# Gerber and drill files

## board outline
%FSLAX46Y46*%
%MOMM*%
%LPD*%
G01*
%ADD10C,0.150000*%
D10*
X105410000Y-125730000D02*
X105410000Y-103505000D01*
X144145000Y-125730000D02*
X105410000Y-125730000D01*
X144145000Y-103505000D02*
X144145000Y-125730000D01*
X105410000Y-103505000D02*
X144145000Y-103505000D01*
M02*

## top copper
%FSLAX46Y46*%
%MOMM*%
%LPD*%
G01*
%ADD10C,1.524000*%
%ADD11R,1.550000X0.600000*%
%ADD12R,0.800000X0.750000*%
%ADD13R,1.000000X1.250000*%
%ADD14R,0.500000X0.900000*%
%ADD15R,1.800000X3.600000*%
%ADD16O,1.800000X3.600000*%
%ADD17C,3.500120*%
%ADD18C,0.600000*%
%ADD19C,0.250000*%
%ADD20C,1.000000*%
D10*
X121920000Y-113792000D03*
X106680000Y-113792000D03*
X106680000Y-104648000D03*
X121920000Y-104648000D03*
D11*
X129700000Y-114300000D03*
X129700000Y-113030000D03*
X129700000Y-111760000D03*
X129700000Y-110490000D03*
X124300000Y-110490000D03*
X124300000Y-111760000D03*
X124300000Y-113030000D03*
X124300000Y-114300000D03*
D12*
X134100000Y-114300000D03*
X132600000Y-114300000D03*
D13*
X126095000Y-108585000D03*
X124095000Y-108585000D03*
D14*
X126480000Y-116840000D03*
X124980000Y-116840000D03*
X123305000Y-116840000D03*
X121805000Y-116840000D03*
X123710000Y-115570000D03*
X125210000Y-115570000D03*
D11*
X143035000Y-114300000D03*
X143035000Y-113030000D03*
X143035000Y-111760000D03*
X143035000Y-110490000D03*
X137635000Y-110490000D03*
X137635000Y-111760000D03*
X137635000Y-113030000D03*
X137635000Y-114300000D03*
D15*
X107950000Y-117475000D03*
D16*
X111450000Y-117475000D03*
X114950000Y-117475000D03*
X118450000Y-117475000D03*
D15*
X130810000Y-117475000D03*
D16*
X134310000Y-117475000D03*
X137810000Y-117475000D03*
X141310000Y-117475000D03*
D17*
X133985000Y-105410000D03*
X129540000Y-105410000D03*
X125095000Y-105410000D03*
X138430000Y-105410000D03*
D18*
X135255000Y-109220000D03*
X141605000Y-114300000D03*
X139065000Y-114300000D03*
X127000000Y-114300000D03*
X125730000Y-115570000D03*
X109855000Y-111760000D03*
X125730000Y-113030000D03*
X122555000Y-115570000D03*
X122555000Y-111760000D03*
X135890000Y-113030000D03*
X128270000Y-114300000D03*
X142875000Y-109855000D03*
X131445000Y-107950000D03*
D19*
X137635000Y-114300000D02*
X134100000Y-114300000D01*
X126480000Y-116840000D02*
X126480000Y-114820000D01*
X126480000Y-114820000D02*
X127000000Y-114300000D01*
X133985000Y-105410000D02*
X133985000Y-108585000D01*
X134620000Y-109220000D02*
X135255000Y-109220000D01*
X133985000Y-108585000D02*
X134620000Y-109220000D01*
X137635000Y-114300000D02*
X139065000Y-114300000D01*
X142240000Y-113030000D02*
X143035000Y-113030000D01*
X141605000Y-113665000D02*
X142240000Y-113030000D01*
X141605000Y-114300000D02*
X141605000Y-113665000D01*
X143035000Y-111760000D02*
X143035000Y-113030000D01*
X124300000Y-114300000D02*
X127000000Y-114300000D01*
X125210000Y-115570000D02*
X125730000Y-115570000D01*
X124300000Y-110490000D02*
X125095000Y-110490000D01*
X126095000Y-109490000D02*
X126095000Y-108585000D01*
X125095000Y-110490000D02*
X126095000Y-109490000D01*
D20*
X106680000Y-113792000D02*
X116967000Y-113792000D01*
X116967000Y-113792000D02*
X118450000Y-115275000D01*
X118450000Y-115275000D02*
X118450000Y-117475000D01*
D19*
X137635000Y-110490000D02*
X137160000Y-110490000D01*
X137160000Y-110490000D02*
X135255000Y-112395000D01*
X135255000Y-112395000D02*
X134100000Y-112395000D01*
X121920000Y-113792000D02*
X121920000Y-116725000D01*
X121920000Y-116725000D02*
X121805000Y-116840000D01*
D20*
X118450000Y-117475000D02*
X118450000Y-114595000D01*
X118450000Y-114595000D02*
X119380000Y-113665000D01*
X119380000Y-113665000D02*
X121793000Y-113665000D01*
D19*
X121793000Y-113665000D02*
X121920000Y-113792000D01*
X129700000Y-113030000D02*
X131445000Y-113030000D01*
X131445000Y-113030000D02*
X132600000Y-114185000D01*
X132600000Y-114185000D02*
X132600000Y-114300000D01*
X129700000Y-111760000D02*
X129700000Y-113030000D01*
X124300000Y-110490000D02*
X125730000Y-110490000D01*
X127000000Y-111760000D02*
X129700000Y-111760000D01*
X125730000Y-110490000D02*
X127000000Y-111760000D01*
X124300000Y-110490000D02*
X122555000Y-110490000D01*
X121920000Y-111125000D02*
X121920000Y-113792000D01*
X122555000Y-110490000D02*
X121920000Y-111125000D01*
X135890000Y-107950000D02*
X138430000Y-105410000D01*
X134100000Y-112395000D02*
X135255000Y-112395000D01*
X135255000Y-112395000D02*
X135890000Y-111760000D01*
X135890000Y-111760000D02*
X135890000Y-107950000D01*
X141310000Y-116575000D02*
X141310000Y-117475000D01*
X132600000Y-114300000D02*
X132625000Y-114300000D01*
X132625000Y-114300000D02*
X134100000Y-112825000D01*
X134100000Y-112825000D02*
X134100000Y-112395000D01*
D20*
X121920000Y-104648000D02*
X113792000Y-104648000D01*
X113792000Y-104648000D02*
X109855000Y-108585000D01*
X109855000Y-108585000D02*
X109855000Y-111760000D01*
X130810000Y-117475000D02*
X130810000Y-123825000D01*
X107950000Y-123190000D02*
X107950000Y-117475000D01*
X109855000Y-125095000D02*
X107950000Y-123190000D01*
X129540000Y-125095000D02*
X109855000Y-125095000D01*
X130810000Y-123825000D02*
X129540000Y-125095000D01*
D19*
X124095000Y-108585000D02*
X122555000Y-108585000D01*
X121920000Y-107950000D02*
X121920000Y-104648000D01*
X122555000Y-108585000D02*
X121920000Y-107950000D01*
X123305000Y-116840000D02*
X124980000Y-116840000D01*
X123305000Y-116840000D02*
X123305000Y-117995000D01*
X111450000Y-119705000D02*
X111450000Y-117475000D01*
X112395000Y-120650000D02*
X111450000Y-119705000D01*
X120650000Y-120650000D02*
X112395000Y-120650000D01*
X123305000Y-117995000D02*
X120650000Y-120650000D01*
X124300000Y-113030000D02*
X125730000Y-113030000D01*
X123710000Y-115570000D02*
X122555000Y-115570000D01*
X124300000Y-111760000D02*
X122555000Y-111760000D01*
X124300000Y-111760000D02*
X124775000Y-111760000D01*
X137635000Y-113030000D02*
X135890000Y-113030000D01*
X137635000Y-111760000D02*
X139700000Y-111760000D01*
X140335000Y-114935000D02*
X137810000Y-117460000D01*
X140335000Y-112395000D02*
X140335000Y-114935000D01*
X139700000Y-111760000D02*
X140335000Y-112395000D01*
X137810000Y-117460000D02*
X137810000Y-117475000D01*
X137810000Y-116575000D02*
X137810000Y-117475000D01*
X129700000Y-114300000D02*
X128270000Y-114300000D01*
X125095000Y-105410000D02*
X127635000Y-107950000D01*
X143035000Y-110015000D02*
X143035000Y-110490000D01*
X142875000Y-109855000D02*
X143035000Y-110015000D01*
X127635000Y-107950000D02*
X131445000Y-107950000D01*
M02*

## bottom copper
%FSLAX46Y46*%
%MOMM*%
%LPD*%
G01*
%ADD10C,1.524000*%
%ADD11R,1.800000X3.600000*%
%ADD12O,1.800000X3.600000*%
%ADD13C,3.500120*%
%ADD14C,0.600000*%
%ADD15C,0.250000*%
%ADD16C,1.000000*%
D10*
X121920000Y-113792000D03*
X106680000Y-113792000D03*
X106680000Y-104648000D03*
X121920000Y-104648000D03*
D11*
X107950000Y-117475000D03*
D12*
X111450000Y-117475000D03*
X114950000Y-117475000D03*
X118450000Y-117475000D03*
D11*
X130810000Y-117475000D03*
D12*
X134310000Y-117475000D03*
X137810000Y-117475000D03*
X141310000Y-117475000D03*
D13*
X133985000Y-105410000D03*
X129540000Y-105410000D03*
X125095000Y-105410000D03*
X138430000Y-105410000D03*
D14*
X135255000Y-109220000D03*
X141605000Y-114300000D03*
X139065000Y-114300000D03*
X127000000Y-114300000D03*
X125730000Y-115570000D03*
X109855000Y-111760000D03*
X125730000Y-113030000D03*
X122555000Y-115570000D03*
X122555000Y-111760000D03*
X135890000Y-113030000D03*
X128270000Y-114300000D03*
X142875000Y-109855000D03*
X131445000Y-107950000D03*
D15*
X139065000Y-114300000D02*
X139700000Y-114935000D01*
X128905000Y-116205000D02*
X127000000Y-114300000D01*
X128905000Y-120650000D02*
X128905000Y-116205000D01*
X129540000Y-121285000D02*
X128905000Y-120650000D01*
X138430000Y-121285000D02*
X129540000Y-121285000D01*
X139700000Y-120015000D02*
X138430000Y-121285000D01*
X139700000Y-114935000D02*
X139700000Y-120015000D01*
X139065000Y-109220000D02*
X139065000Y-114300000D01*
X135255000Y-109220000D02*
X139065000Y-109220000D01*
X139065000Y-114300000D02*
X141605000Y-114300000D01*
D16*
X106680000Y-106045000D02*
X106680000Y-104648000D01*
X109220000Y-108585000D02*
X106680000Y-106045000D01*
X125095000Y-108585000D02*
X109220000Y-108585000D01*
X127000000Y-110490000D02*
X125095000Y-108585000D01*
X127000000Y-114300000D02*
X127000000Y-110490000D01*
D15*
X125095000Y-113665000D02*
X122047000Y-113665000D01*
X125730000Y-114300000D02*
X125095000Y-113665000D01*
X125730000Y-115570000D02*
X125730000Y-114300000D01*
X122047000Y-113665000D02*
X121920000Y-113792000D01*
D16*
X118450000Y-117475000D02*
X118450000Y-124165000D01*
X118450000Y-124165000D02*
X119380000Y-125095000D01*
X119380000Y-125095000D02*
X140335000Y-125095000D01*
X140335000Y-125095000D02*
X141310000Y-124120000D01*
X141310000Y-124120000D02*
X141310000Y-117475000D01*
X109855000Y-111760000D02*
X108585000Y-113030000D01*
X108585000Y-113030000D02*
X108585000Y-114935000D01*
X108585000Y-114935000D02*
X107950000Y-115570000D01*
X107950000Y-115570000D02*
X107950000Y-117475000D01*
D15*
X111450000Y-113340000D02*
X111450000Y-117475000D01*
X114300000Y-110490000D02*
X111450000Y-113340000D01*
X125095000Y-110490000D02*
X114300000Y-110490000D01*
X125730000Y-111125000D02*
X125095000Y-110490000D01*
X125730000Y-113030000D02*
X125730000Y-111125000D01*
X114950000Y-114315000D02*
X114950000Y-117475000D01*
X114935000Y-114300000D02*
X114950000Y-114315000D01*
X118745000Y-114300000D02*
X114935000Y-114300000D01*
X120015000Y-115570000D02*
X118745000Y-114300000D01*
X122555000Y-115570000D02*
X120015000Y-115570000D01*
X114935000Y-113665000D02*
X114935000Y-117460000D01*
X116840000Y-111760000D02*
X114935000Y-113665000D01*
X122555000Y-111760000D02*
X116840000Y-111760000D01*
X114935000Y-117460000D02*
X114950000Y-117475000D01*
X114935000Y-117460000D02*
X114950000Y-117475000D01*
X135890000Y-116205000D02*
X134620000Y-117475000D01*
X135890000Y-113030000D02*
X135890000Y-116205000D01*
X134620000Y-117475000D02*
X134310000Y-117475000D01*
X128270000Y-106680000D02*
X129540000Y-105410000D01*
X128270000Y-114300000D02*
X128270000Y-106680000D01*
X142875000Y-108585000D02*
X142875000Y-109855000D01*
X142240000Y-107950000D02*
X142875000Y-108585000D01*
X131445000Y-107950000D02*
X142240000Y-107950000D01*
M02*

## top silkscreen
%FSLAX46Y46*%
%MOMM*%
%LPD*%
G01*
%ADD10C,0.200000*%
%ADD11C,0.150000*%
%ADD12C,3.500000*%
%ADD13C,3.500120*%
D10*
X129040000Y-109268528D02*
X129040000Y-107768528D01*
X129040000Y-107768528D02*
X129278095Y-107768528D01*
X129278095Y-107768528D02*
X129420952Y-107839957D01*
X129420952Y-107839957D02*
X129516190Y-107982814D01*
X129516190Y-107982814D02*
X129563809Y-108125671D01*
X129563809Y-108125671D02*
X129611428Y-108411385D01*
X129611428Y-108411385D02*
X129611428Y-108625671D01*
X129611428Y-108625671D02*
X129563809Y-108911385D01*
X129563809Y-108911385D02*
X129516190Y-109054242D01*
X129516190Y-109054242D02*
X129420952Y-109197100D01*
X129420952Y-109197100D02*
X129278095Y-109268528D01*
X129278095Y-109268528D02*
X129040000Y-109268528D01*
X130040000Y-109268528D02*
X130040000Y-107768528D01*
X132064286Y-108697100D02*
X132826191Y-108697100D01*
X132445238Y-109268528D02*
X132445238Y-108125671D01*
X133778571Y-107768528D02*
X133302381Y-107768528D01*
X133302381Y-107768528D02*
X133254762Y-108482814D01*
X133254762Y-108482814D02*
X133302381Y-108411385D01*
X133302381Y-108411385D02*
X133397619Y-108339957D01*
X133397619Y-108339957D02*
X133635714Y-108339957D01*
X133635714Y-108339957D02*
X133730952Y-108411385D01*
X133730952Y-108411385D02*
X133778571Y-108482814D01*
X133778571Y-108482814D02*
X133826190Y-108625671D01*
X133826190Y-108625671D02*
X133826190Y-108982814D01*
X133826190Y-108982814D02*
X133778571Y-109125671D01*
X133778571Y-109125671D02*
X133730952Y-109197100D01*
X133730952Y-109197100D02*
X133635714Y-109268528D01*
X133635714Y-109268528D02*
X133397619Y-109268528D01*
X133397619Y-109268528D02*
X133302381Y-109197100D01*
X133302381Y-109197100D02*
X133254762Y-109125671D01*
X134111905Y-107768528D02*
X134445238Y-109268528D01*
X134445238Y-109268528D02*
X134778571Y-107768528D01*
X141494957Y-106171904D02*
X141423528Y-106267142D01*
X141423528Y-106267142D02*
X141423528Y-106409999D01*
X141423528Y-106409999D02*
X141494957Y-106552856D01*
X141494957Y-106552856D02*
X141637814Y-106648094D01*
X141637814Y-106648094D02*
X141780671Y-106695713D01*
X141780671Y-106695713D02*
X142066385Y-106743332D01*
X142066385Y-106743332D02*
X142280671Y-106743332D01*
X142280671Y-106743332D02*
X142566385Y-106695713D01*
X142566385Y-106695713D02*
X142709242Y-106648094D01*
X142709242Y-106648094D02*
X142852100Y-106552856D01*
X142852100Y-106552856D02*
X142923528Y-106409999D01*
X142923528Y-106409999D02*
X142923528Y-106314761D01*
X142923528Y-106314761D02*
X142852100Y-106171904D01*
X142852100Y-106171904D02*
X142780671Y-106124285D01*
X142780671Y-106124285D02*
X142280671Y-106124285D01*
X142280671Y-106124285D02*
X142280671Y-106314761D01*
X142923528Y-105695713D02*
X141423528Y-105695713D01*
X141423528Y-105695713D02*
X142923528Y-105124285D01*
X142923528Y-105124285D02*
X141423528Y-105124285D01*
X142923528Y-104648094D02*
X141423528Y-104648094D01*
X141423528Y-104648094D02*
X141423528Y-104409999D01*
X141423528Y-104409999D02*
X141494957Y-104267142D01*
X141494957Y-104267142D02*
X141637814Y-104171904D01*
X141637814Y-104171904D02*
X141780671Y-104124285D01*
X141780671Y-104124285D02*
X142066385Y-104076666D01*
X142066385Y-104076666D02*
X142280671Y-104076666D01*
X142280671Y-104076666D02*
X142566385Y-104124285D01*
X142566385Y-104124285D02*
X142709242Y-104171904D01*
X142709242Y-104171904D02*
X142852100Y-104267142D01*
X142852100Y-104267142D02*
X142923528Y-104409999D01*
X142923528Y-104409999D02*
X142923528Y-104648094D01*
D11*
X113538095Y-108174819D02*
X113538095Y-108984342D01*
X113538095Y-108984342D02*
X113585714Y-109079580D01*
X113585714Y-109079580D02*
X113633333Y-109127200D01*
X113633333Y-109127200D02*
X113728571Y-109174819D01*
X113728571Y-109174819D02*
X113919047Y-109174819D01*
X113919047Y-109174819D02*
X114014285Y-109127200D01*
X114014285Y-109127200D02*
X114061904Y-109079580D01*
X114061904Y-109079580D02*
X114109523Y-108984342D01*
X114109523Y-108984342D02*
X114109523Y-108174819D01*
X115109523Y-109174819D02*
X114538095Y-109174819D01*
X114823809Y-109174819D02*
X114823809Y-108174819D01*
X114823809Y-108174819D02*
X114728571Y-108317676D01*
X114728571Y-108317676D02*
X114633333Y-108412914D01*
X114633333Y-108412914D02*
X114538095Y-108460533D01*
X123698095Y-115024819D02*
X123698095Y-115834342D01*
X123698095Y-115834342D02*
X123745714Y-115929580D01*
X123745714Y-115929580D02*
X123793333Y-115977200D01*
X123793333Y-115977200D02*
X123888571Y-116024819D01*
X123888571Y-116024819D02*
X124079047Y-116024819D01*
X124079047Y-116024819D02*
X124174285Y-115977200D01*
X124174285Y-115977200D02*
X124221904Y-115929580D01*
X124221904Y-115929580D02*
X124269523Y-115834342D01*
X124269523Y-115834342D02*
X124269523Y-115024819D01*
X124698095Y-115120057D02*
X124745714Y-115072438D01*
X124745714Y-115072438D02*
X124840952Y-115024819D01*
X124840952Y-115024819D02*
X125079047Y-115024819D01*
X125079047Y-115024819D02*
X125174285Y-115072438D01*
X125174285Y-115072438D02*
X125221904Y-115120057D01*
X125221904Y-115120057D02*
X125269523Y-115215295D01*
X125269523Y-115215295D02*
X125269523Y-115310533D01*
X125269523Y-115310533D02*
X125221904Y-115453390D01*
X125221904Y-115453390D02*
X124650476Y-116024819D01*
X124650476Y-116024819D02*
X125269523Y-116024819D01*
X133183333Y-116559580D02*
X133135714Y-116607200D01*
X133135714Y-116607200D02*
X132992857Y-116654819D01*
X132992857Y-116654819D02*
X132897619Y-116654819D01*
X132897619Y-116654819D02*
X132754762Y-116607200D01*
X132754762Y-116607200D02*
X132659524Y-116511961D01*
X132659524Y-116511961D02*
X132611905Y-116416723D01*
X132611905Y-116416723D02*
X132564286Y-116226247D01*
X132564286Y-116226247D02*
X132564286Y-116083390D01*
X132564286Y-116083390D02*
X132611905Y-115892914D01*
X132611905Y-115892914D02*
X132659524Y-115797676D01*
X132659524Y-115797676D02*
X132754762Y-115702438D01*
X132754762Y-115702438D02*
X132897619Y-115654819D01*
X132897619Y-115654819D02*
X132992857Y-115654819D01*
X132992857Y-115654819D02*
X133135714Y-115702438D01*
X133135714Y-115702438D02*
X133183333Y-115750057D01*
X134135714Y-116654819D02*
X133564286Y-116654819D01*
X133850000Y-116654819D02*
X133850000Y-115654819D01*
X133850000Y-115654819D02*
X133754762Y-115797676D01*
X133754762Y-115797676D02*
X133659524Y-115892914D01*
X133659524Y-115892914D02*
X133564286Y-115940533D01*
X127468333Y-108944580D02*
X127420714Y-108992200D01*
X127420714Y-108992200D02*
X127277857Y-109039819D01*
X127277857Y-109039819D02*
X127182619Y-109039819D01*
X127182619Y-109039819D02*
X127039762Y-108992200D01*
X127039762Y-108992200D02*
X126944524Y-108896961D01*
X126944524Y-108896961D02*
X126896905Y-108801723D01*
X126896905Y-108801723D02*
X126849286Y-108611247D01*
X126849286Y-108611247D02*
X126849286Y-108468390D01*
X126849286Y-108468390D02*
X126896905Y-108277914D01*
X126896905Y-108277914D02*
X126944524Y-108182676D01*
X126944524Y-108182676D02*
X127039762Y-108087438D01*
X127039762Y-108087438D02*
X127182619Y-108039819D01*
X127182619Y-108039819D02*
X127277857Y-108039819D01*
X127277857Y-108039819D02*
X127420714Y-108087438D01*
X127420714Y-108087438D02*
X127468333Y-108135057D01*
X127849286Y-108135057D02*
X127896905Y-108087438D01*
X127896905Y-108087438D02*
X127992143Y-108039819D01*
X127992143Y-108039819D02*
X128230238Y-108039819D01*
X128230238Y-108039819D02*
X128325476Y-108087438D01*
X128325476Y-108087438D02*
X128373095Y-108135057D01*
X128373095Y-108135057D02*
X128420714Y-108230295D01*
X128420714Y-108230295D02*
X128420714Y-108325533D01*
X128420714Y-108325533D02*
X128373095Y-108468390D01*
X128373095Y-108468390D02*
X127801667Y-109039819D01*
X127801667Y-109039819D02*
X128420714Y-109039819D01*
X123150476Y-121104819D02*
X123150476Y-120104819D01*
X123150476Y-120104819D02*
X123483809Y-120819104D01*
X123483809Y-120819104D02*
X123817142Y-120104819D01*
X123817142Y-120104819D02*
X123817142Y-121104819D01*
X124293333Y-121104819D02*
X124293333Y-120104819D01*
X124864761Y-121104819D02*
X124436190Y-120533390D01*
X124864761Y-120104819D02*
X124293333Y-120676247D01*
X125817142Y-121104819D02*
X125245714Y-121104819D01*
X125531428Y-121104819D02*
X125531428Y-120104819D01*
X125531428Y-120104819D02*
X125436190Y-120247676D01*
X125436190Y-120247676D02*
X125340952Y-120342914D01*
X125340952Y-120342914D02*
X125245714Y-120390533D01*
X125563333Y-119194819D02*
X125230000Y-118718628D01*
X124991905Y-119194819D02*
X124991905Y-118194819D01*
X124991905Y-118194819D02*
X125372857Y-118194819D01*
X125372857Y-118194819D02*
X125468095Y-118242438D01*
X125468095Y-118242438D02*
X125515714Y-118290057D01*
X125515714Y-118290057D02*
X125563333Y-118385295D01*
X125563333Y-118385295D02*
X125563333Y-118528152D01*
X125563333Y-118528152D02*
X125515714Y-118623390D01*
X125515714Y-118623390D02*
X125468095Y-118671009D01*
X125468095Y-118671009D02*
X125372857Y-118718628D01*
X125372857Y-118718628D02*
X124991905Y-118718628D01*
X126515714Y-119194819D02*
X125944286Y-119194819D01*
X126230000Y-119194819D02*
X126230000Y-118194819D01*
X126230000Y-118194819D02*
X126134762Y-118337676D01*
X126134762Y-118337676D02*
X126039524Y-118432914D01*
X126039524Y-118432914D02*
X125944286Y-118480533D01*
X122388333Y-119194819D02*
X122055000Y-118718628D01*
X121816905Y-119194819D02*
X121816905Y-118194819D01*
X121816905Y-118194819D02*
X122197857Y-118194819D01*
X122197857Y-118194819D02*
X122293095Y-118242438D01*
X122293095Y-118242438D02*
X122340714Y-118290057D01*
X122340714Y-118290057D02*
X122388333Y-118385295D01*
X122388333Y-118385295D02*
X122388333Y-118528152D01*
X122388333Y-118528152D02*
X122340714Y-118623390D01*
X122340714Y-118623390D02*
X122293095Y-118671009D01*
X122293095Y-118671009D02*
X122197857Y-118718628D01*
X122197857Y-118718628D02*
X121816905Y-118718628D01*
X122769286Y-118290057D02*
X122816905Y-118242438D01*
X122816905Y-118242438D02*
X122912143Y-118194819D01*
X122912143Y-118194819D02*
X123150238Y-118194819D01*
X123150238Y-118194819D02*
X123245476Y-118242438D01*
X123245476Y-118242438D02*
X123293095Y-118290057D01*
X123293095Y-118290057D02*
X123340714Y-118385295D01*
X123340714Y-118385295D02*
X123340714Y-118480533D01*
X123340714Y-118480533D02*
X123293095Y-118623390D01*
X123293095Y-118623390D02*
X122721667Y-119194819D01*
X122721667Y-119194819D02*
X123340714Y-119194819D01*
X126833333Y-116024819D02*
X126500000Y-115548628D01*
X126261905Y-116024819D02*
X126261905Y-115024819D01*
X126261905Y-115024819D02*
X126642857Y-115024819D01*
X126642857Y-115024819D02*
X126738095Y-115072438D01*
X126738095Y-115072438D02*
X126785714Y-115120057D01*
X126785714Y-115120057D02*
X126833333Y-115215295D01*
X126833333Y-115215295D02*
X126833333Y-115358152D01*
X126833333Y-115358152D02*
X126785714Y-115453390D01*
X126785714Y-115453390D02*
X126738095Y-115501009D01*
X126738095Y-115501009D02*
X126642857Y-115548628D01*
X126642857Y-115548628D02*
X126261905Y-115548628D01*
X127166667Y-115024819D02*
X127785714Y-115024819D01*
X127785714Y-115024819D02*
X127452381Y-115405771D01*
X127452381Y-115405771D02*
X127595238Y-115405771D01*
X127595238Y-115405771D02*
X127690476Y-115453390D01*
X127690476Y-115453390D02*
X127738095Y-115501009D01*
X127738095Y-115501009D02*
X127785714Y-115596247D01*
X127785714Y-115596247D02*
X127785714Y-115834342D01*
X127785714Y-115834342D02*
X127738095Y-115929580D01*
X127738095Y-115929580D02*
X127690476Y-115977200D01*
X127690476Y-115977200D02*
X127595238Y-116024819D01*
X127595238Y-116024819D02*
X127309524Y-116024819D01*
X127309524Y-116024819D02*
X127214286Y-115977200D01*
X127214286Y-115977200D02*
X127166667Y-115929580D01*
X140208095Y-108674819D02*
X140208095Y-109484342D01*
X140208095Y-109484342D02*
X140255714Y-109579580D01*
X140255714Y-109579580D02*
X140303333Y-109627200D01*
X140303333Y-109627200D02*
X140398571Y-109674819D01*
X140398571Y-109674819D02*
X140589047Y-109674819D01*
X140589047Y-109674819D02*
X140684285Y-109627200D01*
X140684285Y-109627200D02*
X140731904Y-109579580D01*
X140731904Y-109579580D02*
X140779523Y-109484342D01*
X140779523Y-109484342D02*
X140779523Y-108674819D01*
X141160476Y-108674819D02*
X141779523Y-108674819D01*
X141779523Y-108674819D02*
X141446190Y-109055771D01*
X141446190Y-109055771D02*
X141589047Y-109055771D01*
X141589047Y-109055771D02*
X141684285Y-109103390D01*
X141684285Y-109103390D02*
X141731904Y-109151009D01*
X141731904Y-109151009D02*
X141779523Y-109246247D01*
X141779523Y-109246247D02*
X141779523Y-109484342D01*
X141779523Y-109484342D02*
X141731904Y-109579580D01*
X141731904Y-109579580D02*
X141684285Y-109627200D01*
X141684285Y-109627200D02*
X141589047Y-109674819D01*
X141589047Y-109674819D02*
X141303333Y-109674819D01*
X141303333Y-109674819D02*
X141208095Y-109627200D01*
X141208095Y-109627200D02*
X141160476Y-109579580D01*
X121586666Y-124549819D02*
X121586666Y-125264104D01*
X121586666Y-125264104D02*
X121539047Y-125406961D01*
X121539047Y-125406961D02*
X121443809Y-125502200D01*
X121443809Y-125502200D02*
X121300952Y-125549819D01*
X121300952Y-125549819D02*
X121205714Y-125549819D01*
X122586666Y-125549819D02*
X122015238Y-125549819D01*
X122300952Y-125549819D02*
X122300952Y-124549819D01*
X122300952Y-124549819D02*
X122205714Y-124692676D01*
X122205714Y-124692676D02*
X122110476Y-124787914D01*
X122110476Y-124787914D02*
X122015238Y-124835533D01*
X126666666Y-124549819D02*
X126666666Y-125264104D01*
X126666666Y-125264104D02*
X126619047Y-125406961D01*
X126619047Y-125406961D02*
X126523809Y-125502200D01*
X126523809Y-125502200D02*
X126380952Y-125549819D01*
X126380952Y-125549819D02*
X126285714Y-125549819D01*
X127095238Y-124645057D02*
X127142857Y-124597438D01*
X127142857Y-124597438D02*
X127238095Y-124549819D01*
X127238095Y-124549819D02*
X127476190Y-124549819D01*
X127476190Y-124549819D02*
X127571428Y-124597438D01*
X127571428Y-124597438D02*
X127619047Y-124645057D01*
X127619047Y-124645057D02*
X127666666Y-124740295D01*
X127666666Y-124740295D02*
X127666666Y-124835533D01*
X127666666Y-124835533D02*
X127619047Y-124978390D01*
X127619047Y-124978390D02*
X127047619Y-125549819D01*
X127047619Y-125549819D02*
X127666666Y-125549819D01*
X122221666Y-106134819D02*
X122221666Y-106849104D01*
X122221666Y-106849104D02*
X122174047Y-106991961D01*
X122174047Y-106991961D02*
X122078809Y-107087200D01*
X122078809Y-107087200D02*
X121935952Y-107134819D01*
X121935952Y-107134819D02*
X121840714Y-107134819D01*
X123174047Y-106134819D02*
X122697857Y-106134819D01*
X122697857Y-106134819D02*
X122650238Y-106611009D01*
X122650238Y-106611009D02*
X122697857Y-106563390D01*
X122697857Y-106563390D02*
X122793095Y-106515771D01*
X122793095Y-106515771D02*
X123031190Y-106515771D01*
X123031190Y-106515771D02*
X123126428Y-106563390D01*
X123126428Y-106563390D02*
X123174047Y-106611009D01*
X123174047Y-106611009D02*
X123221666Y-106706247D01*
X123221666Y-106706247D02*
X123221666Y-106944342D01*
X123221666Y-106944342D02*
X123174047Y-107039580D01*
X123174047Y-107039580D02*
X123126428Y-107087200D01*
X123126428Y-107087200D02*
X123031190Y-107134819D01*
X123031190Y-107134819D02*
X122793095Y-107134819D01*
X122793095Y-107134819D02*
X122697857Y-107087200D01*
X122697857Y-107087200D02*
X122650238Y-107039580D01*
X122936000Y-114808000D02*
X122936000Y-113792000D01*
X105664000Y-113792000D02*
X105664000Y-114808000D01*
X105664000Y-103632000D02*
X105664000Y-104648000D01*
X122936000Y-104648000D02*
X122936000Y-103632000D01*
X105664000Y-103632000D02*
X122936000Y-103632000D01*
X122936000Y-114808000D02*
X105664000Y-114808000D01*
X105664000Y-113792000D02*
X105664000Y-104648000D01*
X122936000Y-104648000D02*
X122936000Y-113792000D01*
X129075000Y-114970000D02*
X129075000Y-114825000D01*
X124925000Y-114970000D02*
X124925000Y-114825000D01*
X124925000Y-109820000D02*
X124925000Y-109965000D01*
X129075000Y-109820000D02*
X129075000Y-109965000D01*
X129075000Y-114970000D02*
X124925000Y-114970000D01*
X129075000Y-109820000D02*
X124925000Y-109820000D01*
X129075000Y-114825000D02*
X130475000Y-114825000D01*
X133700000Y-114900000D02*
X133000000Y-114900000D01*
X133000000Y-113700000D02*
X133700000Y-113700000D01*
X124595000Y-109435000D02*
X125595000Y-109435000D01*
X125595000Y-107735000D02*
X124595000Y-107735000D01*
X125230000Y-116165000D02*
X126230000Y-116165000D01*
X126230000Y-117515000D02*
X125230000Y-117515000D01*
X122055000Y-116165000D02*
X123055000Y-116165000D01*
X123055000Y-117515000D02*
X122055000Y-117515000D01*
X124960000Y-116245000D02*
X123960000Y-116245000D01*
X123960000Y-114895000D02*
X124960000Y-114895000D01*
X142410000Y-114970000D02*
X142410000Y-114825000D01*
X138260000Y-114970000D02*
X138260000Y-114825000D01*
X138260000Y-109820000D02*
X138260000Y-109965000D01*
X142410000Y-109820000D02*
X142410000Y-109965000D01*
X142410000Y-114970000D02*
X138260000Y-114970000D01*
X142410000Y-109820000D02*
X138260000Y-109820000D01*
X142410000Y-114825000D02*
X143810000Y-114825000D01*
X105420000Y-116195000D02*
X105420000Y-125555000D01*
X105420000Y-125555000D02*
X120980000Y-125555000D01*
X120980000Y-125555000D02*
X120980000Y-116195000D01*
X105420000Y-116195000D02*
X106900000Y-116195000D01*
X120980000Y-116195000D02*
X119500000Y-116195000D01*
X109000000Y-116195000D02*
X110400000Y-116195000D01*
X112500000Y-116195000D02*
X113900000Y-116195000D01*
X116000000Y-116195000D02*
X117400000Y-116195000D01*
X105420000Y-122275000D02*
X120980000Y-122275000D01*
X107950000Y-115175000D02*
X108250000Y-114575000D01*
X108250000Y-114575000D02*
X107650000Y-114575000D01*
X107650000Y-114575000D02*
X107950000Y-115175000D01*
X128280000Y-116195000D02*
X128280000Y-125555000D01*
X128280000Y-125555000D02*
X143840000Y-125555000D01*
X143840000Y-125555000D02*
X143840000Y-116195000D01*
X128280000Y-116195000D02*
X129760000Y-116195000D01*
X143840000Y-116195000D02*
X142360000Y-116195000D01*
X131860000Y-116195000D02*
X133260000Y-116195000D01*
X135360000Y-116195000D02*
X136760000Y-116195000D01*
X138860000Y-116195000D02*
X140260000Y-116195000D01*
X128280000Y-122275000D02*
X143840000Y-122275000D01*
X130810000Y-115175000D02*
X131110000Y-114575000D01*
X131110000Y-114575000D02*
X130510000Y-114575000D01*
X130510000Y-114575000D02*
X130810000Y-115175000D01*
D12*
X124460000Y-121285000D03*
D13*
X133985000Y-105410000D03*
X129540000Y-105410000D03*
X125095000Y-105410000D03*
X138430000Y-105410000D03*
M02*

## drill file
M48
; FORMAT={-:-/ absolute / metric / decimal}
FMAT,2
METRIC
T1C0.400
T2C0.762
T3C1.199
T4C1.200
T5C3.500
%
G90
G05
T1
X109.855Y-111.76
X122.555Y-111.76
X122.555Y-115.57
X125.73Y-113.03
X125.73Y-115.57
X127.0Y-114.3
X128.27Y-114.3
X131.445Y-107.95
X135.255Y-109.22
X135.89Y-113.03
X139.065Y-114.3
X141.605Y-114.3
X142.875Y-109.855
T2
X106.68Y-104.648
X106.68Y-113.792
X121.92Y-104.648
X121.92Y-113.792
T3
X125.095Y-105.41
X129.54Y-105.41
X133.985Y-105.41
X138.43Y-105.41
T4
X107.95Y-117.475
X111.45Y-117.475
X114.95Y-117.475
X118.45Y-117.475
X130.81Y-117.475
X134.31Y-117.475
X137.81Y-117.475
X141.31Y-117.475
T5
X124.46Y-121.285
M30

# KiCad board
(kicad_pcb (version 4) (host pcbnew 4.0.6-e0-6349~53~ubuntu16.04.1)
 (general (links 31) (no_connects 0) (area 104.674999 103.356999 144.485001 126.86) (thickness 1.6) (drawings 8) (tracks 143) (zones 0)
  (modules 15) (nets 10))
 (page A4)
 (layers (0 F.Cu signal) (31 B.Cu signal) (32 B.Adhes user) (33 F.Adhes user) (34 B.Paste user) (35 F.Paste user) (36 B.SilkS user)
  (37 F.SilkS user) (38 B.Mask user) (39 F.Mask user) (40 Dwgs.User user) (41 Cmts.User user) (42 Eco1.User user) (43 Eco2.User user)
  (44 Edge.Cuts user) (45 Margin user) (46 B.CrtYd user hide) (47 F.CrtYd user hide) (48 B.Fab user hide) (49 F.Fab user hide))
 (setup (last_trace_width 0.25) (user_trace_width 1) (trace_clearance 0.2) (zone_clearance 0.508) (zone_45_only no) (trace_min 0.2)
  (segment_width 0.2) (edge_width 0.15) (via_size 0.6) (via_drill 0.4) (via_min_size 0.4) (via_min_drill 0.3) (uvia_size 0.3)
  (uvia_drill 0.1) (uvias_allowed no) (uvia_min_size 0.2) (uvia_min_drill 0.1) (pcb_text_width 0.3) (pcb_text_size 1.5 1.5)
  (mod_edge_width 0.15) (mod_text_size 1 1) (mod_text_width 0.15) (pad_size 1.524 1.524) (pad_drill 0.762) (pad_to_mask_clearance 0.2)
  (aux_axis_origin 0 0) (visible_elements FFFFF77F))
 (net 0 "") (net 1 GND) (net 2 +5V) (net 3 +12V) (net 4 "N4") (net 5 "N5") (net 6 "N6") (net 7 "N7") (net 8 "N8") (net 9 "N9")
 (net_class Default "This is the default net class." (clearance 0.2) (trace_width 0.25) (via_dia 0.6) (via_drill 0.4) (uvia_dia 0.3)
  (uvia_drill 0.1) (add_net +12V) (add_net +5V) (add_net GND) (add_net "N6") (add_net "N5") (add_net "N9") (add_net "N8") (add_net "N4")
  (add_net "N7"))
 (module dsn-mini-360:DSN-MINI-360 (layer F.Cu) (at 114.3 109.22 180)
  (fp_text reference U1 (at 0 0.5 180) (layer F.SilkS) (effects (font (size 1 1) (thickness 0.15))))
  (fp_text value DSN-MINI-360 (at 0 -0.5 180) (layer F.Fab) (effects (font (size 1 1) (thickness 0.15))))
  (fp_line (start -8.636 -5.588) (end -8.636 -4.572) (layer F.SilkS) (width 0.15))
  (fp_line (start 8.636 -4.572) (end 8.636 -5.588) (layer F.SilkS) (width 0.15))
  (fp_line (start 8.636 5.588) (end 8.636 4.572) (layer F.SilkS) (width 0.15))
  (fp_line (start -8.636 4.572) (end -8.636 5.588) (layer F.SilkS) (width 0.15))
  (fp_line (start 8.636 5.588) (end -8.636 5.588) (layer F.SilkS) (width 0.15))
  (fp_line (start -8.636 -5.588) (end 8.636 -5.588) (layer F.SilkS) (width 0.15))
  (fp_line (start 8.636 -4.572) (end 8.636 4.572) (layer F.SilkS) (width 0.15))
  (fp_line (start -8.636 4.572) (end -8.636 -4.572) (layer F.SilkS) (width 0.15))
  (pad IN- thru_hole circle (at -7.62 -4.572 180) (size 1.524 1.524) (drill 0.762) (layers *.Cu *.Mask) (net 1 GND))
  (pad OUT- thru_hole circle (at 7.62 -4.572 180) (size 1.524 1.524) (drill 0.762) (layers *.Cu *.Mask) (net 1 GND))
  (pad OUT+ thru_hole circle (at 7.62 4.572 180) (size 1.524 1.524) (drill 0.762) (layers *.Cu *.Mask) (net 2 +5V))
  (pad IN+ thru_hole circle (at -7.62 4.572 180) (size 1.524 1.524) (drill 0.762) (layers *.Cu *.Mask) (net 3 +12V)))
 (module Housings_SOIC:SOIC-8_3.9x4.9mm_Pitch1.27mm (layer F.Cu) (at 127 112.395 180)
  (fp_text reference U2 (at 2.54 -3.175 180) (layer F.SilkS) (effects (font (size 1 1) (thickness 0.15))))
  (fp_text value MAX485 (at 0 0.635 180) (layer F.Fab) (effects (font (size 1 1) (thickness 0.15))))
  (fp_line (start -2.075 -2.575) (end -2.075 -2.43) (layer F.SilkS) (width 0.15))
  (fp_line (start 2.075 -2.575) (end 2.075 -2.43) (layer F.SilkS) (width 0.15))
  (fp_line (start 2.075 2.575) (end 2.075 2.43) (layer F.SilkS) (width 0.15))
  (fp_line (start -2.075 2.575) (end -2.075 2.43) (layer F.SilkS) (width 0.15))
  (fp_line (start -2.075 -2.575) (end 2.075 -2.575) (layer F.SilkS) (width 0.15))
  (fp_line (start -2.075 2.575) (end 2.075 2.575) (layer F.SilkS) (width 0.15))
  (fp_line (start -2.075 -2.43) (end -3.475 -2.43) (layer F.SilkS) (width 0.15))
  (pad 1 smd rect (at -2.7 -1.905 180) (size 1.55 0.6) (layers F.Cu F.Paste F.Mask) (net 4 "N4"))
  (pad 2 smd rect (at -2.7 -0.635 180) (size 1.55 0.6) (layers F.Cu F.Paste F.Mask) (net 1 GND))
  (pad 3 smd rect (at -2.7 0.635 180) (size 1.55 0.6) (layers F.Cu F.Paste F.Mask) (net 1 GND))
  (pad 4 smd rect (at -2.7 1.905 180) (size 1.55 0.6) (layers F.Cu F.Paste F.Mask))
  (pad 5 smd rect (at 2.7 1.905 180) (size 1.55 0.6) (layers F.Cu F.Paste F.Mask) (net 1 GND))
  (pad 6 smd rect (at 2.7 0.635 180) (size 1.55 0.6) (layers F.Cu F.Paste F.Mask) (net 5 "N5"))
  (pad 7 smd rect (at 2.7 -0.635 180) (size 1.55 0.6) (layers F.Cu F.Paste F.Mask) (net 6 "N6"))
  (pad 8 smd rect (at 2.7 -1.905 180) (size 1.55 0.6) (layers F.Cu F.Paste F.Mask) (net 2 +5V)))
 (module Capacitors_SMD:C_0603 (layer F.Cu) (at 133.35 114.3 180)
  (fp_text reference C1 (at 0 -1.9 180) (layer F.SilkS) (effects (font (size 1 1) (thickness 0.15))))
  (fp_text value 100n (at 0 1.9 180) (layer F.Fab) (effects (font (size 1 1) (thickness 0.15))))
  (fp_line (start -0.35 -0.6) (end 0.35 -0.6) (layer F.SilkS) (width 0.15))
  (fp_line (start 0.35 0.6) (end -0.35 0.6) (layer F.SilkS) (width 0.15))
  (pad 1 smd rect (at -0.75 0 180) (size 0.8 0.75) (layers F.Cu F.Paste F.Mask) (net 2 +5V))
  (pad 2 smd rect (at 0.75 0 180) (size 0.8 0.75) (layers F.Cu F.Paste F.Mask) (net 1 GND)))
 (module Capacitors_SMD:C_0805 (layer F.Cu) (at 125.095 108.585 180)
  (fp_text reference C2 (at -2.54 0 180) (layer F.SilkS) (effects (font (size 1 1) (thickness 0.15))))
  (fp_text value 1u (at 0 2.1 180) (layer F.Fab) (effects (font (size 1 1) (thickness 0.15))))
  (fp_line (start 0.5 -0.85) (end -0.5 -0.85) (layer F.SilkS) (width 0.15))
  (fp_line (start -0.5 0.85) (end 0.5 0.85) (layer F.SilkS) (width 0.15))
  (pad 1 smd rect (at -1 0 180) (size 1 1.25) (layers F.Cu F.Paste F.Mask) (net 1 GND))
  (pad 2 smd rect (at 1 0 180) (size 1 1.25) (layers F.Cu F.Paste F.Mask) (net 3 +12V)))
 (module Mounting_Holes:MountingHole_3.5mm (layer F.Cu) (at 124.46 121.285)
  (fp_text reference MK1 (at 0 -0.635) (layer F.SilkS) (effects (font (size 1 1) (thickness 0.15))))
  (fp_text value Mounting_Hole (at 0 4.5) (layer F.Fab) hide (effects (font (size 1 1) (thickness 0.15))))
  (pad 1 np_thru_hole circle (at 0 0) (size 3.5 3.5) (drill 3.5) (layers *.Cu *.Mask F.SilkS)))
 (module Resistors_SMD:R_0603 (layer F.Cu) (at 125.73 116.84 180)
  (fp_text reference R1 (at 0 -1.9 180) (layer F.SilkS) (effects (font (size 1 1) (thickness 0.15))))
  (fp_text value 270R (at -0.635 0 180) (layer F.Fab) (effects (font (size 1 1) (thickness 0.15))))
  (fp_line (start 0.5 0.675) (end -0.5 0.675) (layer F.SilkS) (width 0.15))
  (fp_line (start -0.5 -0.675) (end 0.5 -0.675) (layer F.SilkS) (width 0.15))
  (pad 1 smd rect (at -0.75 0 180) (size 0.5 0.9) (layers F.Cu F.Paste F.Mask) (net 2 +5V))
  (pad 2 smd rect (at 0.75 0 180) (size 0.5 0.9) (layers F.Cu F.Paste F.Mask) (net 6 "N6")))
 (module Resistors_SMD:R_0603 (layer F.Cu) (at 122.555 116.84 180)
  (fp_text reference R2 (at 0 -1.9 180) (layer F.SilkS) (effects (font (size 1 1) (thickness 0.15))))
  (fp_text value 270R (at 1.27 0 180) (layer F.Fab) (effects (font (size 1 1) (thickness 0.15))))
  (fp_line (start 0.5 0.675) (end -0.5 0.675) (layer F.SilkS) (width 0.15))
  (fp_line (start -0.5 -0.675) (end 0.5 -0.675) (layer F.SilkS) (width 0.15))
  (pad 1 smd rect (at -0.75 0 180) (size 0.5 0.9) (layers F.Cu F.Paste F.Mask) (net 6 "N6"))
  (pad 2 smd rect (at 0.75 0 180) (size 0.5 0.9) (layers F.Cu F.Paste F.Mask) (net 1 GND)))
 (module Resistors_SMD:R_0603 (layer F.Cu) (at 124.46 115.57)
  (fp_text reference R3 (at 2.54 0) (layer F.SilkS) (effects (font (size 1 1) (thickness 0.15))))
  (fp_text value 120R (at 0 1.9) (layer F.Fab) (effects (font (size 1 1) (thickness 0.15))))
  (fp_line (start 0.5 0.675) (end -0.5 0.675) (layer F.SilkS) (width 0.15))
  (fp_line (start -0.5 -0.675) (end 0.5 -0.675) (layer F.SilkS) (width 0.15))
  (pad 1 smd rect (at -0.75 0) (size 0.5 0.9) (layers F.Cu F.Paste F.Mask) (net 5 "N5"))
  (pad 2 smd rect (at 0.75 0) (size 0.5 0.9) (layers F.Cu F.Paste F.Mask) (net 1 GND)))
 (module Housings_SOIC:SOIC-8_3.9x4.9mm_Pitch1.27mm (layer F.Cu) (at 140.335 112.395 180)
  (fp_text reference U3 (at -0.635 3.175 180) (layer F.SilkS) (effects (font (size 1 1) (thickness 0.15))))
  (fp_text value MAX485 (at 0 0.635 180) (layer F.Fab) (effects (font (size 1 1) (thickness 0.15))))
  (fp_line (start -2.075 -2.575) (end -2.075 -2.43) (layer F.SilkS) (width 0.15))
  (fp_line (start 2.075 -2.575) (end 2.075 -2.43) (layer F.SilkS) (width 0.15))
  (fp_line (start 2.075 2.575) (end 2.075 2.43) (layer F.SilkS) (width 0.15))
  (fp_line (start -2.075 2.575) (end -2.075 2.43) (layer F.SilkS) (width 0.15))
  (fp_line (start -2.075 -2.575) (end 2.075 -2.575) (layer F.SilkS) (width 0.15))
  (fp_line (start -2.075 2.575) (end 2.075 2.575) (layer F.SilkS) (width 0.15))
  (fp_line (start -2.075 -2.43) (end -3.475 -2.43) (layer F.SilkS) (width 0.15))
  (pad 1 smd rect (at -2.7 -1.905 180) (size 1.55 0.6) (layers F.Cu F.Paste F.Mask))
  (pad 2 smd rect (at -2.7 -0.635 180) (size 1.55 0.6) (layers F.Cu F.Paste F.Mask) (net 2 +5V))
  (pad 3 smd rect (at -2.7 0.635 180) (size 1.55 0.6) (layers F.Cu F.Paste F.Mask) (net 2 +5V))
  (pad 4 smd rect (at -2.7 1.905 180) (size 1.55 0.6) (layers F.Cu F.Paste F.Mask) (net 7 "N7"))
  (pad 5 smd rect (at 2.7 1.905 180) (size 1.55 0.6) (layers F.Cu F.Paste F.Mask) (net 1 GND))
  (pad 6 smd rect (at 2.7 0.635 180) (size 1.55 0.6) (layers F.Cu F.Paste F.Mask) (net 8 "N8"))
  (pad 7 smd rect (at 2.7 -0.635 180) (size 1.55 0.6) (layers F.Cu F.Paste F.Mask) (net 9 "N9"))
  (pad 8 smd rect (at 2.7 -1.905 180) (size 1.55 0.6) (layers F.Cu F.Paste F.Mask) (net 2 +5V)))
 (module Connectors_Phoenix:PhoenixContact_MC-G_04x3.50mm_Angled (layer F.Cu) (at 107.95 117.475)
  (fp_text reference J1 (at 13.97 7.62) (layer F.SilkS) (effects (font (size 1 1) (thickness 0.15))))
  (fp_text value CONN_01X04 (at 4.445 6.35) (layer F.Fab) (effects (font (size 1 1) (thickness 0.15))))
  (fp_line (start -2.53 -1.28) (end -2.53 8.08) (layer F.SilkS) (width 0.15))
  (fp_line (start -2.53 8.08) (end 13.03 8.08) (layer F.SilkS) (width 0.15))
  (fp_line (start 13.03 8.08) (end 13.03 -1.28) (layer F.SilkS) (width 0.15))
  (fp_line (start -2.53 -1.28) (end -1.05 -1.28) (layer F.SilkS) (width 0.15))
  (fp_line (start 13.03 -1.28) (end 11.55 -1.28) (layer F.SilkS) (width 0.15))
  (fp_line (start 1.05 -1.28) (end 2.45 -1.28) (layer F.SilkS) (width 0.15))
  (fp_line (start 4.55 -1.28) (end 5.95 -1.28) (layer F.SilkS) (width 0.15))
  (fp_line (start 8.05 -1.28) (end 9.45 -1.28) (layer F.SilkS) (width 0.15))
  (fp_line (start -2.53 4.8) (end 13.03 4.8) (layer F.SilkS) (width 0.15))
  (fp_line (start 0 -2.3) (end 0.3 -2.9) (layer F.SilkS) (width 0.15))
  (fp_line (start 0.3 -2.9) (end -0.3 -2.9) (layer F.SilkS) (width 0.15))
  (fp_line (start -0.3 -2.9) (end 0 -2.3) (layer F.SilkS) (width 0.15))
  (pad 1 thru_hole rect (at 0 0) (size 1.8 3.6) (drill 1.2) (layers *.Cu *.Mask) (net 3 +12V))
  (pad 2 thru_hole oval (at 3.5 0) (size 1.8 3.6) (drill 1.2) (layers *.Cu *.Mask) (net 6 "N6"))
  (pad 3 thru_hole oval (at 7 0) (size 1.8 3.6) (drill 1.2) (layers *.Cu *.Mask) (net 5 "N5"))
  (pad 4 thru_hole oval (at 10.5 0) (size 1.8 3.6) (drill 1.2) (layers *.Cu *.Mask) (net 1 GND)))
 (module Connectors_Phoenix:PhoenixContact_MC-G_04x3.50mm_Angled (layer F.Cu) (at 130.81 117.475)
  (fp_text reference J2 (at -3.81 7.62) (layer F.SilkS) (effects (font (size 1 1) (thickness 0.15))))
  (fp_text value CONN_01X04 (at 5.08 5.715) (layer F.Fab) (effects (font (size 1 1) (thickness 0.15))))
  (fp_line (start -2.53 -1.28) (end -2.53 8.08) (layer F.SilkS) (width 0.15))
  (fp_line (start -2.53 8.08) (end 13.03 8.08) (layer F.SilkS) (width 0.15))
  (fp_line (start 13.03 8.08) (end 13.03 -1.28) (layer F.SilkS) (width 0.15))
  (fp_line (start -2.53 -1.28) (end -1.05 -1.28) (layer F.SilkS) (width 0.15))
  (fp_line (start 13.03 -1.28) (end 11.55 -1.28) (layer F.SilkS) (width 0.15))
  (fp_line (start 1.05 -1.28) (end 2.45 -1.28) (layer F.SilkS) (width 0.15))
  (fp_line (start 4.55 -1.28) (end 5.95 -1.28) (layer F.SilkS) (width 0.15))
  (fp_line (start 8.05 -1.28) (end 9.45 -1.28) (layer F.SilkS) (width 0.15))
  (fp_line (start -2.53 4.8) (end 13.03 4.8) (layer F.SilkS) (width 0.15))
  (fp_line (start 0 -2.3) (end 0.3 -2.9) (layer F.SilkS) (width 0.15))
  (fp_line (start 0.3 -2.9) (end -0.3 -2.9) (layer F.SilkS) (width 0.15))
  (fp_line (start -0.3 -2.9) (end 0 -2.3) (layer F.SilkS) (width 0.15))
  (pad 1 thru_hole rect (at 0 0) (size 1.8 3.6) (drill 1.2) (layers *.Cu *.Mask) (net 3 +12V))
  (pad 2 thru_hole oval (at 3.5 0) (size 1.8 3.6) (drill 1.2) (layers *.Cu *.Mask) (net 9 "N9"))
  (pad 3 thru_hole oval (at 7 0) (size 1.8 3.6) (drill 1.2) (layers *.Cu *.Mask) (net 8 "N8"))
  (pad 4 thru_hole oval (at 10.5 0) (size 1.8 3.6) (drill 1.2) (layers *.Cu *.Mask) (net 1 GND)))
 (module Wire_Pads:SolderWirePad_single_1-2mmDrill (layer F.Cu) (at 133.985 105.41)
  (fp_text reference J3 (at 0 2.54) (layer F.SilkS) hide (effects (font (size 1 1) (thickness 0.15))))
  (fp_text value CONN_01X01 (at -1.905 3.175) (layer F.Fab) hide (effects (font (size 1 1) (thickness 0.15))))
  (pad 1 thru_hole circle (at 0 0) (size 3.50012 3.50012) (drill 1.19888) (layers *.Cu *.Mask F.SilkS) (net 2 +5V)))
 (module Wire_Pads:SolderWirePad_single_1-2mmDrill (layer F.Cu) (at 129.54 105.41)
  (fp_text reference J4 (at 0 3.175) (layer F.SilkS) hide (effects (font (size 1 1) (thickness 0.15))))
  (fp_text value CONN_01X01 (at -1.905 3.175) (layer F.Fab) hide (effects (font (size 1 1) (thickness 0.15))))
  (pad 1 thru_hole circle (at 0 0) (size 3.50012 3.50012) (drill 1.19888) (layers *.Cu *.Mask F.SilkS) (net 4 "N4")))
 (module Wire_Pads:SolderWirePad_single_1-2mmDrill (layer F.Cu) (at 125.095 105.41)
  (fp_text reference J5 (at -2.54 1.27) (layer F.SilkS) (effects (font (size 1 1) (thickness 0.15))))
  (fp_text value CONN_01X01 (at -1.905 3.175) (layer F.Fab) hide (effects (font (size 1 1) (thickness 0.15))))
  (pad 1 thru_hole circle (at 0 0) (size 3.50012 3.50012) (drill 1.19888) (layers *.Cu *.Mask F.SilkS) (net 7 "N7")))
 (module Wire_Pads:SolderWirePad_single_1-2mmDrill (layer F.Cu) (at 138.43 105.41)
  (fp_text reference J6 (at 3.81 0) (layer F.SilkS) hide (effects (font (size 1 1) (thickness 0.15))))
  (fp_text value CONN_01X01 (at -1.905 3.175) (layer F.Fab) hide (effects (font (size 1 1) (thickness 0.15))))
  (pad 1 thru_hole circle (at 0 0) (size 3.50012 3.50012) (drill 1.19888) (layers *.Cu *.Mask F.SilkS) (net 1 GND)))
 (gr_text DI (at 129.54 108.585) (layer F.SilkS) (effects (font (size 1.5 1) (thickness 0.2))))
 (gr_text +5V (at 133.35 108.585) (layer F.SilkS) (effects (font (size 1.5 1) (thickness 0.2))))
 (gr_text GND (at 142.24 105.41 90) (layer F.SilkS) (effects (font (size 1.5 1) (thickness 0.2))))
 (gr_line (start 105.41 125.73) (end 105.41 103.505) (angle 90) (layer Edge.Cuts) (width 0.15))
 (gr_line (start 144.145 125.73) (end 105.41 125.73) (angle 90) (layer Edge.Cuts) (width 0.15))
 (gr_line (start 144.145 103.505) (end 144.145 125.73) (angle 90) (layer Edge.Cuts) (width 0.15))
 (gr_line (start 105.41 103.505) (end 144.145 103.505) (angle 90) (layer Edge.Cuts) (width 0.15))
 (segment (start 137.635 114.3) (end 134.1 114.3) (width 0.25) (layer F.Cu) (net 2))
 (segment (start 139.065 114.3) (end 139.7 114.935) (width 0.25) (layer B.Cu) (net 2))
 (segment (start 128.905 116.205) (end 127 114.3) (width 0.25) (layer B.Cu) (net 2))
 (segment (start 128.905 120.65) (end 128.905 116.205) (width 0.25) (layer B.Cu) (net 2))
 (segment (start 129.54 121.285) (end 128.905 120.65) (width 0.25) (layer B.Cu) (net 2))
 (segment (start 138.43 121.285) (end 129.54 121.285) (width 0.25) (layer B.Cu) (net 2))
 (segment (start 139.7 120.015) (end 138.43 121.285) (width 0.25) (layer B.Cu) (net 2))
 (segment (start 139.7 114.935) (end 139.7 120.015) (width 0.25) (layer B.Cu) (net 2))
 (segment (start 126.48 116.84) (end 126.48 114.82) (width 0.25) (layer F.Cu) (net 2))
 (segment (start 126.48 114.82) (end 127 114.3) (width 0.25) (layer F.Cu) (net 2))
 (segment (start 133.985 105.41) (end 133.985 108.585) (width 0.25) (layer F.Cu) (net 2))
 (segment (start 139.065 109.22) (end 139.065 114.3) (width 0.25) (layer B.Cu) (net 2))
 (segment (start 135.255 109.22) (end 139.065 109.22) (width 0.25) (layer B.Cu) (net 2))
 (via (at 135.255 109.22) (size 0.6) (drill 0.4) (layers F.Cu B.Cu) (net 2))
 (segment (start 134.62 109.22) (end 135.255 109.22) (width 0.25) (layer F.Cu) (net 2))
 (segment (start 133.985 108.585) (end 134.62 109.22) (width 0.25) (layer F.Cu) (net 2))
 (segment (start 137.635 114.3) (end 139.065 114.3) (width 0.25) (layer F.Cu) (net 2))
 (segment (start 142.24 113.03) (end 143.035 113.03) (width 0.25) (layer F.Cu) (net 2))
 (segment (start 141.605 113.665) (end 142.24 113.03) (width 0.25) (layer F.Cu) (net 2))
 (segment (start 141.605 114.3) (end 141.605 113.665) (width 0.25) (layer F.Cu) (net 2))
 (via (at 141.605 114.3) (size 0.6) (drill 0.4) (layers F.Cu B.Cu) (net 2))
 (segment (start 139.065 114.3) (end 141.605 114.3) (width 0.25) (layer B.Cu) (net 2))
 (via (at 139.065 114.3) (size 0.6) (drill 0.4) (layers F.Cu B.Cu) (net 2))
 (segment (start 143.035 111.76) (end 143.035 113.03) (width 0.25) (layer F.Cu) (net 2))
 (segment (start 124.3 114.3) (end 127 114.3) (width 0.25) (layer F.Cu) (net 2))
 (segment (start 106.68 106.045) (end 106.68 104.648) (width 1) (layer B.Cu) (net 2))
 (segment (start 109.22 108.585) (end 106.68 106.045) (width 1) (layer B.Cu) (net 2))
 (segment (start 125.095 108.585) (end 109.22 108.585) (width 1) (layer B.Cu) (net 2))
 (segment (start 127 110.49) (end 125.095 108.585) (width 1) (layer B.Cu) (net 2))
 (segment (start 127 114.3) (end 127 110.49) (width 1) (layer B.Cu) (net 2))
 (via (at 127 114.3) (size 0.6) (drill 0.4) (layers F.Cu B.Cu) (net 2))
 (segment (start 125.21 115.57) (end 125.73 115.57) (width 0.25) (layer F.Cu) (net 1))
 (segment (start 125.095 113.665) (end 122.047 113.665) (width 0.25) (layer B.Cu) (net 1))
 (segment (start 125.73 114.3) (end 125.095 113.665) (width 0.25) (layer B.Cu) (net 1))
 (segment (start 125.73 115.57) (end 125.73 114.3) (width 0.25) (layer B.Cu) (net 1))
 (via (at 125.73 115.57) (size 0.6) (drill 0.4) (layers F.Cu B.Cu) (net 1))
 (segment (start 122.047 113.665) (end 121.92 113.792) (width 0.25) (layer B.Cu) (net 1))
 (segment (start 124.3 110.49) (end 125.095 110.49) (width 0.25) (layer F.Cu) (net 1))
 (segment (start 126.095 109.49) (end 126.095 108.585) (width 0.25) (layer F.Cu) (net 1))
 (segment (start 125.095 110.49) (end 126.095 109.49) (width 0.25) (layer F.Cu) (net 1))
 (segment (start 106.68 113.792) (end 116.967 113.792) (width 1) (layer F.Cu) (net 1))
 (segment (start 116.967 113.792) (end 118.45 115.275) (width 1) (layer F.Cu) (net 1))
 (segment (start 118.45 115.275) (end 118.45 117.475) (width 1) (layer F.Cu) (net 1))
 (segment (start 137.635 110.49) (end 137.16 110.49) (width 0.25) (layer F.Cu) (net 1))
 (segment (start 137.16 110.49) (end 135.255 112.395) (width 0.25) (layer F.Cu) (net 1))
 (segment (start 135.255 112.395) (end 134.1 112.395) (width 0.25) (layer F.Cu) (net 1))
 (segment (start 118.45 117.475) (end 118.45 124.165) (width 1) (layer B.Cu) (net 1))
 (segment (start 118.45 124.165) (end 119.38 125.095) (width 1) (layer B.Cu) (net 1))
 (segment (start 119.38 125.095) (end 140.335 125.095) (width 1) (layer B.Cu) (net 1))
 (segment (start 140.335 125.095) (end 141.31 124.12) (width 1) (layer B.Cu) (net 1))
 (segment (start 141.31 124.12) (end 141.31 117.475) (width 1) (layer B.Cu) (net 1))
 (segment (start 121.92 113.792) (end 121.92 116.725) (width 0.25) (layer F.Cu) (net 1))
 (segment (start 121.92 116.725) (end 121.805 116.84) (width 0.25) (layer F.Cu) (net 1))
 (segment (start 118.45 117.475) (end 118.45 114.595) (width 1) (layer F.Cu) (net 1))
 (segment (start 118.45 114.595) (end 119.38 113.665) (width 1) (layer F.Cu) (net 1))
 (segment (start 119.38 113.665) (end 121.793 113.665) (width 1) (layer F.Cu) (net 1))
 (segment (start 121.793 113.665) (end 121.92 113.792) (width 0.25) (layer F.Cu) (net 1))
 (segment (start 129.7 113.03) (end 131.445 113.03) (width 0.25) (layer F.Cu) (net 1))
 (segment (start 131.445 113.03) (end 132.6 114.185) (width 0.25) (layer F.Cu) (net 1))
 (segment (start 132.6 114.185) (end 132.6 114.3) (width 0.25) (layer F.Cu) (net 1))
 (segment (start 129.7 111.76) (end 129.7 113.03) (width 0.25) (layer F.Cu) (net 1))
 (segment (start 124.3 110.49) (end 125.73 110.49) (width 0.25) (layer F.Cu) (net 1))
 (segment (start 127 111.76) (end 129.7 111.76) (width 0.25) (layer F.Cu) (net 1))
 (segment (start 125.73 110.49) (end 127 111.76) (width 0.25) (layer F.Cu) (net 1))
 (segment (start 124.3 110.49) (end 122.555 110.49) (width 0.25) (layer F.Cu) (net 1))
 (segment (start 121.92 111.125) (end 121.92 113.792) (width 0.25) (layer F.Cu) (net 1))
 (segment (start 122.555 110.49) (end 121.92 111.125) (width 0.25) (layer F.Cu) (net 1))
 (segment (start 135.89 107.95) (end 138.43 105.41) (width 0.25) (layer F.Cu) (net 1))
 (segment (start 134.1 112.395) (end 135.255 112.395) (width 0.25) (layer F.Cu) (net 1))
 (segment (start 135.255 112.395) (end 135.89 111.76) (width 0.25) (layer F.Cu) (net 1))
 (segment (start 135.89 111.76) (end 135.89 107.95) (width 0.25) (layer F.Cu) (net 1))
 (segment (start 141.31 116.575) (end 141.31 117.475) (width 0.25) (layer F.Cu) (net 1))
 (segment (start 132.6 114.3) (end 132.625 114.3) (width 0.25) (layer F.Cu) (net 1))
 (segment (start 132.625 114.3) (end 134.1 112.825) (width 0.25) (layer F.Cu) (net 1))
 (segment (start 134.1 112.825) (end 134.1 112.395) (width 0.25) (layer F.Cu) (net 1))
 (segment (start 121.92 104.648) (end 113.792 104.648) (width 1) (layer F.Cu) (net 3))
 (segment (start 113.792 104.648) (end 109.855 108.585) (width 1) (layer F.Cu) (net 3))
 (segment (start 109.855 108.585) (end 109.855 111.76) (width 1) (layer F.Cu) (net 3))
 (via (at 109.855 111.76) (size 0.6) (drill 0.4) (layers F.Cu B.Cu) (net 3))
 (segment (start 109.855 111.76) (end 108.585 113.03) (width 1) (layer B.Cu) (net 3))
 (segment (start 108.585 113.03) (end 108.585 114.935) (width 1) (layer B.Cu) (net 3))
 (segment (start 108.585 114.935) (end 107.95 115.57) (width 1) (layer B.Cu) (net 3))
 (segment (start 107.95 115.57) (end 107.95 117.475) (width 1) (layer B.Cu) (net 3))
 (segment (start 130.81 117.475) (end 130.81 123.825) (width 1) (layer F.Cu) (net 3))
 (segment (start 107.95 123.19) (end 107.95 117.475) (width 1) (layer F.Cu) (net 3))
 (segment (start 109.855 125.095) (end 107.95 123.19) (width 1) (layer F.Cu) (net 3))
 (segment (start 129.54 125.095) (end 109.855 125.095) (width 1) (layer F.Cu) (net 3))
 (segment (start 130.81 123.825) (end 129.54 125.095) (width 1) (layer F.Cu) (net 3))
 (segment (start 124.095 108.585) (end 122.555 108.585) (width 0.25) (layer F.Cu) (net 3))
 (segment (start 121.92 107.95) (end 121.92 104.648) (width 0.25) (layer F.Cu) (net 3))
 (segment (start 122.555 108.585) (end 121.92 107.95) (width 0.25) (layer F.Cu) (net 3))
 (segment (start 123.305 116.84) (end 124.98 116.84) (width 0.25) (layer F.Cu) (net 6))
 (segment (start 123.305 116.84) (end 123.305 117.995) (width 0.25) (layer F.Cu) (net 6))
 (segment (start 111.45 119.705) (end 111.45 117.475) (width 0.25) (layer F.Cu) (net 6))
 (segment (start 112.395 120.65) (end 111.45 119.705) (width 0.25) (layer F.Cu) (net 6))
 (segment (start 120.65 120.65) (end 112.395 120.65) (width 0.25) (layer F.Cu) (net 6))
 (segment (start 123.305 117.995) (end 120.65 120.65) (width 0.25) (layer F.Cu) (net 6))
 (segment (start 124.3 113.03) (end 125.73 113.03) (width 0.25) (layer F.Cu) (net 6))
 (segment (start 111.45 113.34) (end 111.45 117.475) (width 0.25) (layer B.Cu) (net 6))
 (segment (start 114.3 110.49) (end 111.45 113.34) (width 0.25) (layer B.Cu) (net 6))
 (segment (start 125.095 110.49) (end 114.3 110.49) (width 0.25) (layer B.Cu) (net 6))
 (segment (start 125.73 111.125) (end 125.095 110.49) (width 0.25) (layer B.Cu) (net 6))
 (segment (start 125.73 113.03) (end 125.73 111.125) (width 0.25) (layer B.Cu) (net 6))
 (via (at 125.73 113.03) (size 0.6) (drill 0.4) (layers F.Cu B.Cu) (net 6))
 (segment (start 123.71 115.57) (end 122.555 115.57) (width 0.25) (layer F.Cu) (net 5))
 (segment (start 114.95 114.315) (end 114.95 117.475) (width 0.25) (layer B.Cu) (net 5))
 (segment (start 114.935 114.3) (end 114.95 114.315) (width 0.25) (layer B.Cu) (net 5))
 (segment (start 118.745 114.3) (end 114.935 114.3) (width 0.25) (layer B.Cu) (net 5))
 (segment (start 120.015 115.57) (end 118.745 114.3) (width 0.25) (layer B.Cu) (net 5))
 (segment (start 122.555 115.57) (end 120.015 115.57) (width 0.25) (layer B.Cu) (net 5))
 (via (at 122.555 115.57) (size 0.6) (drill 0.4) (layers F.Cu B.Cu) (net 5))
 (segment (start 124.3 111.76) (end 122.555 111.76) (width 0.25) (layer F.Cu) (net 5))
 (segment (start 114.935 113.665) (end 114.935 117.46) (width 0.25) (layer B.Cu) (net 5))
 (segment (start 116.84 111.76) (end 114.935 113.665) (width 0.25) (layer B.Cu) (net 5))
 (segment (start 122.555 111.76) (end 116.84 111.76) (width 0.25) (layer B.Cu) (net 5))
 (via (at 122.555 111.76) (size 0.6) (drill 0.4) (layers F.Cu B.Cu) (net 5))
 (segment (start 114.935 117.46) (end 114.95 117.475) (width 0.25) (layer B.Cu) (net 5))
 (segment (start 114.935 117.46) (end 114.95 117.475) (width 0.25) (layer B.Cu) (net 5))
 (segment (start 124.3 111.76) (end 124.775 111.76) (width 0.25) (layer F.Cu) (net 5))
 (segment (start 137.635 113.03) (end 135.89 113.03) (width 0.25) (layer F.Cu) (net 9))
 (segment (start 135.89 116.205) (end 134.62 117.475) (width 0.25) (layer B.Cu) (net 9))
 (segment (start 135.89 113.03) (end 135.89 116.205) (width 0.25) (layer B.Cu) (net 9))
 (via (at 135.89 113.03) (size 0.6) (drill 0.4) (layers F.Cu B.Cu) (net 9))
 (segment (start 134.62 117.475) (end 134.31 117.475) (width 0.25) (layer B.Cu) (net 9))
 (segment (start 137.635 111.76) (end 139.7 111.76) (width 0.25) (layer F.Cu) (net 8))
 (segment (start 140.335 114.935) (end 137.81 117.46) (width 0.25) (layer F.Cu) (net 8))
 (segment (start 140.335 112.395) (end 140.335 114.935) (width 0.25) (layer F.Cu) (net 8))
 (segment (start 139.7 111.76) (end 140.335 112.395) (width 0.25) (layer F.Cu) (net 8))
 (segment (start 137.81 117.46) (end 137.81 117.475) (width 0.25) (layer F.Cu) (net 8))
 (segment (start 137.81 116.575) (end 137.81 117.475) (width 0.25) (layer F.Cu) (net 8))
 (segment (start 129.7 114.3) (end 128.27 114.3) (width 0.25) (layer F.Cu) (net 4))
 (segment (start 128.27 106.68) (end 129.54 105.41) (width 0.25) (layer B.Cu) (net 4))
 (segment (start 128.27 114.3) (end 128.27 106.68) (width 0.25) (layer B.Cu) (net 4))
 (via (at 128.27 114.3) (size 0.6) (drill 0.4) (layers F.Cu B.Cu) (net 4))
 (segment (start 125.095 105.41) (end 127.635 107.95) (width 0.25) (layer F.Cu) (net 7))
 (segment (start 143.035 110.015) (end 143.035 110.49) (width 0.25) (layer F.Cu) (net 7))
 (segment (start 142.875 109.855) (end 143.035 110.015) (width 0.25) (layer F.Cu) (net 7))
 (via (at 142.875 109.855) (size 0.6) (drill 0.4) (layers F.Cu B.Cu) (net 7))
 (segment (start 142.875 108.585) (end 142.875 109.855) (width 0.25) (layer B.Cu) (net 7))
 (segment (start 142.24 107.95) (end 142.875 108.585) (width 0.25) (layer B.Cu) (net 7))
 (segment (start 131.445 107.95) (end 142.24 107.95) (width 0.25) (layer B.Cu) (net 7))
 (via (at 131.445 107.95) (size 0.6) (drill 0.4) (layers F.Cu B.Cu) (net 7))
 (segment (start 127.635 107.95) (end 131.445 107.95) (width 0.25) (layer F.Cu) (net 7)))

